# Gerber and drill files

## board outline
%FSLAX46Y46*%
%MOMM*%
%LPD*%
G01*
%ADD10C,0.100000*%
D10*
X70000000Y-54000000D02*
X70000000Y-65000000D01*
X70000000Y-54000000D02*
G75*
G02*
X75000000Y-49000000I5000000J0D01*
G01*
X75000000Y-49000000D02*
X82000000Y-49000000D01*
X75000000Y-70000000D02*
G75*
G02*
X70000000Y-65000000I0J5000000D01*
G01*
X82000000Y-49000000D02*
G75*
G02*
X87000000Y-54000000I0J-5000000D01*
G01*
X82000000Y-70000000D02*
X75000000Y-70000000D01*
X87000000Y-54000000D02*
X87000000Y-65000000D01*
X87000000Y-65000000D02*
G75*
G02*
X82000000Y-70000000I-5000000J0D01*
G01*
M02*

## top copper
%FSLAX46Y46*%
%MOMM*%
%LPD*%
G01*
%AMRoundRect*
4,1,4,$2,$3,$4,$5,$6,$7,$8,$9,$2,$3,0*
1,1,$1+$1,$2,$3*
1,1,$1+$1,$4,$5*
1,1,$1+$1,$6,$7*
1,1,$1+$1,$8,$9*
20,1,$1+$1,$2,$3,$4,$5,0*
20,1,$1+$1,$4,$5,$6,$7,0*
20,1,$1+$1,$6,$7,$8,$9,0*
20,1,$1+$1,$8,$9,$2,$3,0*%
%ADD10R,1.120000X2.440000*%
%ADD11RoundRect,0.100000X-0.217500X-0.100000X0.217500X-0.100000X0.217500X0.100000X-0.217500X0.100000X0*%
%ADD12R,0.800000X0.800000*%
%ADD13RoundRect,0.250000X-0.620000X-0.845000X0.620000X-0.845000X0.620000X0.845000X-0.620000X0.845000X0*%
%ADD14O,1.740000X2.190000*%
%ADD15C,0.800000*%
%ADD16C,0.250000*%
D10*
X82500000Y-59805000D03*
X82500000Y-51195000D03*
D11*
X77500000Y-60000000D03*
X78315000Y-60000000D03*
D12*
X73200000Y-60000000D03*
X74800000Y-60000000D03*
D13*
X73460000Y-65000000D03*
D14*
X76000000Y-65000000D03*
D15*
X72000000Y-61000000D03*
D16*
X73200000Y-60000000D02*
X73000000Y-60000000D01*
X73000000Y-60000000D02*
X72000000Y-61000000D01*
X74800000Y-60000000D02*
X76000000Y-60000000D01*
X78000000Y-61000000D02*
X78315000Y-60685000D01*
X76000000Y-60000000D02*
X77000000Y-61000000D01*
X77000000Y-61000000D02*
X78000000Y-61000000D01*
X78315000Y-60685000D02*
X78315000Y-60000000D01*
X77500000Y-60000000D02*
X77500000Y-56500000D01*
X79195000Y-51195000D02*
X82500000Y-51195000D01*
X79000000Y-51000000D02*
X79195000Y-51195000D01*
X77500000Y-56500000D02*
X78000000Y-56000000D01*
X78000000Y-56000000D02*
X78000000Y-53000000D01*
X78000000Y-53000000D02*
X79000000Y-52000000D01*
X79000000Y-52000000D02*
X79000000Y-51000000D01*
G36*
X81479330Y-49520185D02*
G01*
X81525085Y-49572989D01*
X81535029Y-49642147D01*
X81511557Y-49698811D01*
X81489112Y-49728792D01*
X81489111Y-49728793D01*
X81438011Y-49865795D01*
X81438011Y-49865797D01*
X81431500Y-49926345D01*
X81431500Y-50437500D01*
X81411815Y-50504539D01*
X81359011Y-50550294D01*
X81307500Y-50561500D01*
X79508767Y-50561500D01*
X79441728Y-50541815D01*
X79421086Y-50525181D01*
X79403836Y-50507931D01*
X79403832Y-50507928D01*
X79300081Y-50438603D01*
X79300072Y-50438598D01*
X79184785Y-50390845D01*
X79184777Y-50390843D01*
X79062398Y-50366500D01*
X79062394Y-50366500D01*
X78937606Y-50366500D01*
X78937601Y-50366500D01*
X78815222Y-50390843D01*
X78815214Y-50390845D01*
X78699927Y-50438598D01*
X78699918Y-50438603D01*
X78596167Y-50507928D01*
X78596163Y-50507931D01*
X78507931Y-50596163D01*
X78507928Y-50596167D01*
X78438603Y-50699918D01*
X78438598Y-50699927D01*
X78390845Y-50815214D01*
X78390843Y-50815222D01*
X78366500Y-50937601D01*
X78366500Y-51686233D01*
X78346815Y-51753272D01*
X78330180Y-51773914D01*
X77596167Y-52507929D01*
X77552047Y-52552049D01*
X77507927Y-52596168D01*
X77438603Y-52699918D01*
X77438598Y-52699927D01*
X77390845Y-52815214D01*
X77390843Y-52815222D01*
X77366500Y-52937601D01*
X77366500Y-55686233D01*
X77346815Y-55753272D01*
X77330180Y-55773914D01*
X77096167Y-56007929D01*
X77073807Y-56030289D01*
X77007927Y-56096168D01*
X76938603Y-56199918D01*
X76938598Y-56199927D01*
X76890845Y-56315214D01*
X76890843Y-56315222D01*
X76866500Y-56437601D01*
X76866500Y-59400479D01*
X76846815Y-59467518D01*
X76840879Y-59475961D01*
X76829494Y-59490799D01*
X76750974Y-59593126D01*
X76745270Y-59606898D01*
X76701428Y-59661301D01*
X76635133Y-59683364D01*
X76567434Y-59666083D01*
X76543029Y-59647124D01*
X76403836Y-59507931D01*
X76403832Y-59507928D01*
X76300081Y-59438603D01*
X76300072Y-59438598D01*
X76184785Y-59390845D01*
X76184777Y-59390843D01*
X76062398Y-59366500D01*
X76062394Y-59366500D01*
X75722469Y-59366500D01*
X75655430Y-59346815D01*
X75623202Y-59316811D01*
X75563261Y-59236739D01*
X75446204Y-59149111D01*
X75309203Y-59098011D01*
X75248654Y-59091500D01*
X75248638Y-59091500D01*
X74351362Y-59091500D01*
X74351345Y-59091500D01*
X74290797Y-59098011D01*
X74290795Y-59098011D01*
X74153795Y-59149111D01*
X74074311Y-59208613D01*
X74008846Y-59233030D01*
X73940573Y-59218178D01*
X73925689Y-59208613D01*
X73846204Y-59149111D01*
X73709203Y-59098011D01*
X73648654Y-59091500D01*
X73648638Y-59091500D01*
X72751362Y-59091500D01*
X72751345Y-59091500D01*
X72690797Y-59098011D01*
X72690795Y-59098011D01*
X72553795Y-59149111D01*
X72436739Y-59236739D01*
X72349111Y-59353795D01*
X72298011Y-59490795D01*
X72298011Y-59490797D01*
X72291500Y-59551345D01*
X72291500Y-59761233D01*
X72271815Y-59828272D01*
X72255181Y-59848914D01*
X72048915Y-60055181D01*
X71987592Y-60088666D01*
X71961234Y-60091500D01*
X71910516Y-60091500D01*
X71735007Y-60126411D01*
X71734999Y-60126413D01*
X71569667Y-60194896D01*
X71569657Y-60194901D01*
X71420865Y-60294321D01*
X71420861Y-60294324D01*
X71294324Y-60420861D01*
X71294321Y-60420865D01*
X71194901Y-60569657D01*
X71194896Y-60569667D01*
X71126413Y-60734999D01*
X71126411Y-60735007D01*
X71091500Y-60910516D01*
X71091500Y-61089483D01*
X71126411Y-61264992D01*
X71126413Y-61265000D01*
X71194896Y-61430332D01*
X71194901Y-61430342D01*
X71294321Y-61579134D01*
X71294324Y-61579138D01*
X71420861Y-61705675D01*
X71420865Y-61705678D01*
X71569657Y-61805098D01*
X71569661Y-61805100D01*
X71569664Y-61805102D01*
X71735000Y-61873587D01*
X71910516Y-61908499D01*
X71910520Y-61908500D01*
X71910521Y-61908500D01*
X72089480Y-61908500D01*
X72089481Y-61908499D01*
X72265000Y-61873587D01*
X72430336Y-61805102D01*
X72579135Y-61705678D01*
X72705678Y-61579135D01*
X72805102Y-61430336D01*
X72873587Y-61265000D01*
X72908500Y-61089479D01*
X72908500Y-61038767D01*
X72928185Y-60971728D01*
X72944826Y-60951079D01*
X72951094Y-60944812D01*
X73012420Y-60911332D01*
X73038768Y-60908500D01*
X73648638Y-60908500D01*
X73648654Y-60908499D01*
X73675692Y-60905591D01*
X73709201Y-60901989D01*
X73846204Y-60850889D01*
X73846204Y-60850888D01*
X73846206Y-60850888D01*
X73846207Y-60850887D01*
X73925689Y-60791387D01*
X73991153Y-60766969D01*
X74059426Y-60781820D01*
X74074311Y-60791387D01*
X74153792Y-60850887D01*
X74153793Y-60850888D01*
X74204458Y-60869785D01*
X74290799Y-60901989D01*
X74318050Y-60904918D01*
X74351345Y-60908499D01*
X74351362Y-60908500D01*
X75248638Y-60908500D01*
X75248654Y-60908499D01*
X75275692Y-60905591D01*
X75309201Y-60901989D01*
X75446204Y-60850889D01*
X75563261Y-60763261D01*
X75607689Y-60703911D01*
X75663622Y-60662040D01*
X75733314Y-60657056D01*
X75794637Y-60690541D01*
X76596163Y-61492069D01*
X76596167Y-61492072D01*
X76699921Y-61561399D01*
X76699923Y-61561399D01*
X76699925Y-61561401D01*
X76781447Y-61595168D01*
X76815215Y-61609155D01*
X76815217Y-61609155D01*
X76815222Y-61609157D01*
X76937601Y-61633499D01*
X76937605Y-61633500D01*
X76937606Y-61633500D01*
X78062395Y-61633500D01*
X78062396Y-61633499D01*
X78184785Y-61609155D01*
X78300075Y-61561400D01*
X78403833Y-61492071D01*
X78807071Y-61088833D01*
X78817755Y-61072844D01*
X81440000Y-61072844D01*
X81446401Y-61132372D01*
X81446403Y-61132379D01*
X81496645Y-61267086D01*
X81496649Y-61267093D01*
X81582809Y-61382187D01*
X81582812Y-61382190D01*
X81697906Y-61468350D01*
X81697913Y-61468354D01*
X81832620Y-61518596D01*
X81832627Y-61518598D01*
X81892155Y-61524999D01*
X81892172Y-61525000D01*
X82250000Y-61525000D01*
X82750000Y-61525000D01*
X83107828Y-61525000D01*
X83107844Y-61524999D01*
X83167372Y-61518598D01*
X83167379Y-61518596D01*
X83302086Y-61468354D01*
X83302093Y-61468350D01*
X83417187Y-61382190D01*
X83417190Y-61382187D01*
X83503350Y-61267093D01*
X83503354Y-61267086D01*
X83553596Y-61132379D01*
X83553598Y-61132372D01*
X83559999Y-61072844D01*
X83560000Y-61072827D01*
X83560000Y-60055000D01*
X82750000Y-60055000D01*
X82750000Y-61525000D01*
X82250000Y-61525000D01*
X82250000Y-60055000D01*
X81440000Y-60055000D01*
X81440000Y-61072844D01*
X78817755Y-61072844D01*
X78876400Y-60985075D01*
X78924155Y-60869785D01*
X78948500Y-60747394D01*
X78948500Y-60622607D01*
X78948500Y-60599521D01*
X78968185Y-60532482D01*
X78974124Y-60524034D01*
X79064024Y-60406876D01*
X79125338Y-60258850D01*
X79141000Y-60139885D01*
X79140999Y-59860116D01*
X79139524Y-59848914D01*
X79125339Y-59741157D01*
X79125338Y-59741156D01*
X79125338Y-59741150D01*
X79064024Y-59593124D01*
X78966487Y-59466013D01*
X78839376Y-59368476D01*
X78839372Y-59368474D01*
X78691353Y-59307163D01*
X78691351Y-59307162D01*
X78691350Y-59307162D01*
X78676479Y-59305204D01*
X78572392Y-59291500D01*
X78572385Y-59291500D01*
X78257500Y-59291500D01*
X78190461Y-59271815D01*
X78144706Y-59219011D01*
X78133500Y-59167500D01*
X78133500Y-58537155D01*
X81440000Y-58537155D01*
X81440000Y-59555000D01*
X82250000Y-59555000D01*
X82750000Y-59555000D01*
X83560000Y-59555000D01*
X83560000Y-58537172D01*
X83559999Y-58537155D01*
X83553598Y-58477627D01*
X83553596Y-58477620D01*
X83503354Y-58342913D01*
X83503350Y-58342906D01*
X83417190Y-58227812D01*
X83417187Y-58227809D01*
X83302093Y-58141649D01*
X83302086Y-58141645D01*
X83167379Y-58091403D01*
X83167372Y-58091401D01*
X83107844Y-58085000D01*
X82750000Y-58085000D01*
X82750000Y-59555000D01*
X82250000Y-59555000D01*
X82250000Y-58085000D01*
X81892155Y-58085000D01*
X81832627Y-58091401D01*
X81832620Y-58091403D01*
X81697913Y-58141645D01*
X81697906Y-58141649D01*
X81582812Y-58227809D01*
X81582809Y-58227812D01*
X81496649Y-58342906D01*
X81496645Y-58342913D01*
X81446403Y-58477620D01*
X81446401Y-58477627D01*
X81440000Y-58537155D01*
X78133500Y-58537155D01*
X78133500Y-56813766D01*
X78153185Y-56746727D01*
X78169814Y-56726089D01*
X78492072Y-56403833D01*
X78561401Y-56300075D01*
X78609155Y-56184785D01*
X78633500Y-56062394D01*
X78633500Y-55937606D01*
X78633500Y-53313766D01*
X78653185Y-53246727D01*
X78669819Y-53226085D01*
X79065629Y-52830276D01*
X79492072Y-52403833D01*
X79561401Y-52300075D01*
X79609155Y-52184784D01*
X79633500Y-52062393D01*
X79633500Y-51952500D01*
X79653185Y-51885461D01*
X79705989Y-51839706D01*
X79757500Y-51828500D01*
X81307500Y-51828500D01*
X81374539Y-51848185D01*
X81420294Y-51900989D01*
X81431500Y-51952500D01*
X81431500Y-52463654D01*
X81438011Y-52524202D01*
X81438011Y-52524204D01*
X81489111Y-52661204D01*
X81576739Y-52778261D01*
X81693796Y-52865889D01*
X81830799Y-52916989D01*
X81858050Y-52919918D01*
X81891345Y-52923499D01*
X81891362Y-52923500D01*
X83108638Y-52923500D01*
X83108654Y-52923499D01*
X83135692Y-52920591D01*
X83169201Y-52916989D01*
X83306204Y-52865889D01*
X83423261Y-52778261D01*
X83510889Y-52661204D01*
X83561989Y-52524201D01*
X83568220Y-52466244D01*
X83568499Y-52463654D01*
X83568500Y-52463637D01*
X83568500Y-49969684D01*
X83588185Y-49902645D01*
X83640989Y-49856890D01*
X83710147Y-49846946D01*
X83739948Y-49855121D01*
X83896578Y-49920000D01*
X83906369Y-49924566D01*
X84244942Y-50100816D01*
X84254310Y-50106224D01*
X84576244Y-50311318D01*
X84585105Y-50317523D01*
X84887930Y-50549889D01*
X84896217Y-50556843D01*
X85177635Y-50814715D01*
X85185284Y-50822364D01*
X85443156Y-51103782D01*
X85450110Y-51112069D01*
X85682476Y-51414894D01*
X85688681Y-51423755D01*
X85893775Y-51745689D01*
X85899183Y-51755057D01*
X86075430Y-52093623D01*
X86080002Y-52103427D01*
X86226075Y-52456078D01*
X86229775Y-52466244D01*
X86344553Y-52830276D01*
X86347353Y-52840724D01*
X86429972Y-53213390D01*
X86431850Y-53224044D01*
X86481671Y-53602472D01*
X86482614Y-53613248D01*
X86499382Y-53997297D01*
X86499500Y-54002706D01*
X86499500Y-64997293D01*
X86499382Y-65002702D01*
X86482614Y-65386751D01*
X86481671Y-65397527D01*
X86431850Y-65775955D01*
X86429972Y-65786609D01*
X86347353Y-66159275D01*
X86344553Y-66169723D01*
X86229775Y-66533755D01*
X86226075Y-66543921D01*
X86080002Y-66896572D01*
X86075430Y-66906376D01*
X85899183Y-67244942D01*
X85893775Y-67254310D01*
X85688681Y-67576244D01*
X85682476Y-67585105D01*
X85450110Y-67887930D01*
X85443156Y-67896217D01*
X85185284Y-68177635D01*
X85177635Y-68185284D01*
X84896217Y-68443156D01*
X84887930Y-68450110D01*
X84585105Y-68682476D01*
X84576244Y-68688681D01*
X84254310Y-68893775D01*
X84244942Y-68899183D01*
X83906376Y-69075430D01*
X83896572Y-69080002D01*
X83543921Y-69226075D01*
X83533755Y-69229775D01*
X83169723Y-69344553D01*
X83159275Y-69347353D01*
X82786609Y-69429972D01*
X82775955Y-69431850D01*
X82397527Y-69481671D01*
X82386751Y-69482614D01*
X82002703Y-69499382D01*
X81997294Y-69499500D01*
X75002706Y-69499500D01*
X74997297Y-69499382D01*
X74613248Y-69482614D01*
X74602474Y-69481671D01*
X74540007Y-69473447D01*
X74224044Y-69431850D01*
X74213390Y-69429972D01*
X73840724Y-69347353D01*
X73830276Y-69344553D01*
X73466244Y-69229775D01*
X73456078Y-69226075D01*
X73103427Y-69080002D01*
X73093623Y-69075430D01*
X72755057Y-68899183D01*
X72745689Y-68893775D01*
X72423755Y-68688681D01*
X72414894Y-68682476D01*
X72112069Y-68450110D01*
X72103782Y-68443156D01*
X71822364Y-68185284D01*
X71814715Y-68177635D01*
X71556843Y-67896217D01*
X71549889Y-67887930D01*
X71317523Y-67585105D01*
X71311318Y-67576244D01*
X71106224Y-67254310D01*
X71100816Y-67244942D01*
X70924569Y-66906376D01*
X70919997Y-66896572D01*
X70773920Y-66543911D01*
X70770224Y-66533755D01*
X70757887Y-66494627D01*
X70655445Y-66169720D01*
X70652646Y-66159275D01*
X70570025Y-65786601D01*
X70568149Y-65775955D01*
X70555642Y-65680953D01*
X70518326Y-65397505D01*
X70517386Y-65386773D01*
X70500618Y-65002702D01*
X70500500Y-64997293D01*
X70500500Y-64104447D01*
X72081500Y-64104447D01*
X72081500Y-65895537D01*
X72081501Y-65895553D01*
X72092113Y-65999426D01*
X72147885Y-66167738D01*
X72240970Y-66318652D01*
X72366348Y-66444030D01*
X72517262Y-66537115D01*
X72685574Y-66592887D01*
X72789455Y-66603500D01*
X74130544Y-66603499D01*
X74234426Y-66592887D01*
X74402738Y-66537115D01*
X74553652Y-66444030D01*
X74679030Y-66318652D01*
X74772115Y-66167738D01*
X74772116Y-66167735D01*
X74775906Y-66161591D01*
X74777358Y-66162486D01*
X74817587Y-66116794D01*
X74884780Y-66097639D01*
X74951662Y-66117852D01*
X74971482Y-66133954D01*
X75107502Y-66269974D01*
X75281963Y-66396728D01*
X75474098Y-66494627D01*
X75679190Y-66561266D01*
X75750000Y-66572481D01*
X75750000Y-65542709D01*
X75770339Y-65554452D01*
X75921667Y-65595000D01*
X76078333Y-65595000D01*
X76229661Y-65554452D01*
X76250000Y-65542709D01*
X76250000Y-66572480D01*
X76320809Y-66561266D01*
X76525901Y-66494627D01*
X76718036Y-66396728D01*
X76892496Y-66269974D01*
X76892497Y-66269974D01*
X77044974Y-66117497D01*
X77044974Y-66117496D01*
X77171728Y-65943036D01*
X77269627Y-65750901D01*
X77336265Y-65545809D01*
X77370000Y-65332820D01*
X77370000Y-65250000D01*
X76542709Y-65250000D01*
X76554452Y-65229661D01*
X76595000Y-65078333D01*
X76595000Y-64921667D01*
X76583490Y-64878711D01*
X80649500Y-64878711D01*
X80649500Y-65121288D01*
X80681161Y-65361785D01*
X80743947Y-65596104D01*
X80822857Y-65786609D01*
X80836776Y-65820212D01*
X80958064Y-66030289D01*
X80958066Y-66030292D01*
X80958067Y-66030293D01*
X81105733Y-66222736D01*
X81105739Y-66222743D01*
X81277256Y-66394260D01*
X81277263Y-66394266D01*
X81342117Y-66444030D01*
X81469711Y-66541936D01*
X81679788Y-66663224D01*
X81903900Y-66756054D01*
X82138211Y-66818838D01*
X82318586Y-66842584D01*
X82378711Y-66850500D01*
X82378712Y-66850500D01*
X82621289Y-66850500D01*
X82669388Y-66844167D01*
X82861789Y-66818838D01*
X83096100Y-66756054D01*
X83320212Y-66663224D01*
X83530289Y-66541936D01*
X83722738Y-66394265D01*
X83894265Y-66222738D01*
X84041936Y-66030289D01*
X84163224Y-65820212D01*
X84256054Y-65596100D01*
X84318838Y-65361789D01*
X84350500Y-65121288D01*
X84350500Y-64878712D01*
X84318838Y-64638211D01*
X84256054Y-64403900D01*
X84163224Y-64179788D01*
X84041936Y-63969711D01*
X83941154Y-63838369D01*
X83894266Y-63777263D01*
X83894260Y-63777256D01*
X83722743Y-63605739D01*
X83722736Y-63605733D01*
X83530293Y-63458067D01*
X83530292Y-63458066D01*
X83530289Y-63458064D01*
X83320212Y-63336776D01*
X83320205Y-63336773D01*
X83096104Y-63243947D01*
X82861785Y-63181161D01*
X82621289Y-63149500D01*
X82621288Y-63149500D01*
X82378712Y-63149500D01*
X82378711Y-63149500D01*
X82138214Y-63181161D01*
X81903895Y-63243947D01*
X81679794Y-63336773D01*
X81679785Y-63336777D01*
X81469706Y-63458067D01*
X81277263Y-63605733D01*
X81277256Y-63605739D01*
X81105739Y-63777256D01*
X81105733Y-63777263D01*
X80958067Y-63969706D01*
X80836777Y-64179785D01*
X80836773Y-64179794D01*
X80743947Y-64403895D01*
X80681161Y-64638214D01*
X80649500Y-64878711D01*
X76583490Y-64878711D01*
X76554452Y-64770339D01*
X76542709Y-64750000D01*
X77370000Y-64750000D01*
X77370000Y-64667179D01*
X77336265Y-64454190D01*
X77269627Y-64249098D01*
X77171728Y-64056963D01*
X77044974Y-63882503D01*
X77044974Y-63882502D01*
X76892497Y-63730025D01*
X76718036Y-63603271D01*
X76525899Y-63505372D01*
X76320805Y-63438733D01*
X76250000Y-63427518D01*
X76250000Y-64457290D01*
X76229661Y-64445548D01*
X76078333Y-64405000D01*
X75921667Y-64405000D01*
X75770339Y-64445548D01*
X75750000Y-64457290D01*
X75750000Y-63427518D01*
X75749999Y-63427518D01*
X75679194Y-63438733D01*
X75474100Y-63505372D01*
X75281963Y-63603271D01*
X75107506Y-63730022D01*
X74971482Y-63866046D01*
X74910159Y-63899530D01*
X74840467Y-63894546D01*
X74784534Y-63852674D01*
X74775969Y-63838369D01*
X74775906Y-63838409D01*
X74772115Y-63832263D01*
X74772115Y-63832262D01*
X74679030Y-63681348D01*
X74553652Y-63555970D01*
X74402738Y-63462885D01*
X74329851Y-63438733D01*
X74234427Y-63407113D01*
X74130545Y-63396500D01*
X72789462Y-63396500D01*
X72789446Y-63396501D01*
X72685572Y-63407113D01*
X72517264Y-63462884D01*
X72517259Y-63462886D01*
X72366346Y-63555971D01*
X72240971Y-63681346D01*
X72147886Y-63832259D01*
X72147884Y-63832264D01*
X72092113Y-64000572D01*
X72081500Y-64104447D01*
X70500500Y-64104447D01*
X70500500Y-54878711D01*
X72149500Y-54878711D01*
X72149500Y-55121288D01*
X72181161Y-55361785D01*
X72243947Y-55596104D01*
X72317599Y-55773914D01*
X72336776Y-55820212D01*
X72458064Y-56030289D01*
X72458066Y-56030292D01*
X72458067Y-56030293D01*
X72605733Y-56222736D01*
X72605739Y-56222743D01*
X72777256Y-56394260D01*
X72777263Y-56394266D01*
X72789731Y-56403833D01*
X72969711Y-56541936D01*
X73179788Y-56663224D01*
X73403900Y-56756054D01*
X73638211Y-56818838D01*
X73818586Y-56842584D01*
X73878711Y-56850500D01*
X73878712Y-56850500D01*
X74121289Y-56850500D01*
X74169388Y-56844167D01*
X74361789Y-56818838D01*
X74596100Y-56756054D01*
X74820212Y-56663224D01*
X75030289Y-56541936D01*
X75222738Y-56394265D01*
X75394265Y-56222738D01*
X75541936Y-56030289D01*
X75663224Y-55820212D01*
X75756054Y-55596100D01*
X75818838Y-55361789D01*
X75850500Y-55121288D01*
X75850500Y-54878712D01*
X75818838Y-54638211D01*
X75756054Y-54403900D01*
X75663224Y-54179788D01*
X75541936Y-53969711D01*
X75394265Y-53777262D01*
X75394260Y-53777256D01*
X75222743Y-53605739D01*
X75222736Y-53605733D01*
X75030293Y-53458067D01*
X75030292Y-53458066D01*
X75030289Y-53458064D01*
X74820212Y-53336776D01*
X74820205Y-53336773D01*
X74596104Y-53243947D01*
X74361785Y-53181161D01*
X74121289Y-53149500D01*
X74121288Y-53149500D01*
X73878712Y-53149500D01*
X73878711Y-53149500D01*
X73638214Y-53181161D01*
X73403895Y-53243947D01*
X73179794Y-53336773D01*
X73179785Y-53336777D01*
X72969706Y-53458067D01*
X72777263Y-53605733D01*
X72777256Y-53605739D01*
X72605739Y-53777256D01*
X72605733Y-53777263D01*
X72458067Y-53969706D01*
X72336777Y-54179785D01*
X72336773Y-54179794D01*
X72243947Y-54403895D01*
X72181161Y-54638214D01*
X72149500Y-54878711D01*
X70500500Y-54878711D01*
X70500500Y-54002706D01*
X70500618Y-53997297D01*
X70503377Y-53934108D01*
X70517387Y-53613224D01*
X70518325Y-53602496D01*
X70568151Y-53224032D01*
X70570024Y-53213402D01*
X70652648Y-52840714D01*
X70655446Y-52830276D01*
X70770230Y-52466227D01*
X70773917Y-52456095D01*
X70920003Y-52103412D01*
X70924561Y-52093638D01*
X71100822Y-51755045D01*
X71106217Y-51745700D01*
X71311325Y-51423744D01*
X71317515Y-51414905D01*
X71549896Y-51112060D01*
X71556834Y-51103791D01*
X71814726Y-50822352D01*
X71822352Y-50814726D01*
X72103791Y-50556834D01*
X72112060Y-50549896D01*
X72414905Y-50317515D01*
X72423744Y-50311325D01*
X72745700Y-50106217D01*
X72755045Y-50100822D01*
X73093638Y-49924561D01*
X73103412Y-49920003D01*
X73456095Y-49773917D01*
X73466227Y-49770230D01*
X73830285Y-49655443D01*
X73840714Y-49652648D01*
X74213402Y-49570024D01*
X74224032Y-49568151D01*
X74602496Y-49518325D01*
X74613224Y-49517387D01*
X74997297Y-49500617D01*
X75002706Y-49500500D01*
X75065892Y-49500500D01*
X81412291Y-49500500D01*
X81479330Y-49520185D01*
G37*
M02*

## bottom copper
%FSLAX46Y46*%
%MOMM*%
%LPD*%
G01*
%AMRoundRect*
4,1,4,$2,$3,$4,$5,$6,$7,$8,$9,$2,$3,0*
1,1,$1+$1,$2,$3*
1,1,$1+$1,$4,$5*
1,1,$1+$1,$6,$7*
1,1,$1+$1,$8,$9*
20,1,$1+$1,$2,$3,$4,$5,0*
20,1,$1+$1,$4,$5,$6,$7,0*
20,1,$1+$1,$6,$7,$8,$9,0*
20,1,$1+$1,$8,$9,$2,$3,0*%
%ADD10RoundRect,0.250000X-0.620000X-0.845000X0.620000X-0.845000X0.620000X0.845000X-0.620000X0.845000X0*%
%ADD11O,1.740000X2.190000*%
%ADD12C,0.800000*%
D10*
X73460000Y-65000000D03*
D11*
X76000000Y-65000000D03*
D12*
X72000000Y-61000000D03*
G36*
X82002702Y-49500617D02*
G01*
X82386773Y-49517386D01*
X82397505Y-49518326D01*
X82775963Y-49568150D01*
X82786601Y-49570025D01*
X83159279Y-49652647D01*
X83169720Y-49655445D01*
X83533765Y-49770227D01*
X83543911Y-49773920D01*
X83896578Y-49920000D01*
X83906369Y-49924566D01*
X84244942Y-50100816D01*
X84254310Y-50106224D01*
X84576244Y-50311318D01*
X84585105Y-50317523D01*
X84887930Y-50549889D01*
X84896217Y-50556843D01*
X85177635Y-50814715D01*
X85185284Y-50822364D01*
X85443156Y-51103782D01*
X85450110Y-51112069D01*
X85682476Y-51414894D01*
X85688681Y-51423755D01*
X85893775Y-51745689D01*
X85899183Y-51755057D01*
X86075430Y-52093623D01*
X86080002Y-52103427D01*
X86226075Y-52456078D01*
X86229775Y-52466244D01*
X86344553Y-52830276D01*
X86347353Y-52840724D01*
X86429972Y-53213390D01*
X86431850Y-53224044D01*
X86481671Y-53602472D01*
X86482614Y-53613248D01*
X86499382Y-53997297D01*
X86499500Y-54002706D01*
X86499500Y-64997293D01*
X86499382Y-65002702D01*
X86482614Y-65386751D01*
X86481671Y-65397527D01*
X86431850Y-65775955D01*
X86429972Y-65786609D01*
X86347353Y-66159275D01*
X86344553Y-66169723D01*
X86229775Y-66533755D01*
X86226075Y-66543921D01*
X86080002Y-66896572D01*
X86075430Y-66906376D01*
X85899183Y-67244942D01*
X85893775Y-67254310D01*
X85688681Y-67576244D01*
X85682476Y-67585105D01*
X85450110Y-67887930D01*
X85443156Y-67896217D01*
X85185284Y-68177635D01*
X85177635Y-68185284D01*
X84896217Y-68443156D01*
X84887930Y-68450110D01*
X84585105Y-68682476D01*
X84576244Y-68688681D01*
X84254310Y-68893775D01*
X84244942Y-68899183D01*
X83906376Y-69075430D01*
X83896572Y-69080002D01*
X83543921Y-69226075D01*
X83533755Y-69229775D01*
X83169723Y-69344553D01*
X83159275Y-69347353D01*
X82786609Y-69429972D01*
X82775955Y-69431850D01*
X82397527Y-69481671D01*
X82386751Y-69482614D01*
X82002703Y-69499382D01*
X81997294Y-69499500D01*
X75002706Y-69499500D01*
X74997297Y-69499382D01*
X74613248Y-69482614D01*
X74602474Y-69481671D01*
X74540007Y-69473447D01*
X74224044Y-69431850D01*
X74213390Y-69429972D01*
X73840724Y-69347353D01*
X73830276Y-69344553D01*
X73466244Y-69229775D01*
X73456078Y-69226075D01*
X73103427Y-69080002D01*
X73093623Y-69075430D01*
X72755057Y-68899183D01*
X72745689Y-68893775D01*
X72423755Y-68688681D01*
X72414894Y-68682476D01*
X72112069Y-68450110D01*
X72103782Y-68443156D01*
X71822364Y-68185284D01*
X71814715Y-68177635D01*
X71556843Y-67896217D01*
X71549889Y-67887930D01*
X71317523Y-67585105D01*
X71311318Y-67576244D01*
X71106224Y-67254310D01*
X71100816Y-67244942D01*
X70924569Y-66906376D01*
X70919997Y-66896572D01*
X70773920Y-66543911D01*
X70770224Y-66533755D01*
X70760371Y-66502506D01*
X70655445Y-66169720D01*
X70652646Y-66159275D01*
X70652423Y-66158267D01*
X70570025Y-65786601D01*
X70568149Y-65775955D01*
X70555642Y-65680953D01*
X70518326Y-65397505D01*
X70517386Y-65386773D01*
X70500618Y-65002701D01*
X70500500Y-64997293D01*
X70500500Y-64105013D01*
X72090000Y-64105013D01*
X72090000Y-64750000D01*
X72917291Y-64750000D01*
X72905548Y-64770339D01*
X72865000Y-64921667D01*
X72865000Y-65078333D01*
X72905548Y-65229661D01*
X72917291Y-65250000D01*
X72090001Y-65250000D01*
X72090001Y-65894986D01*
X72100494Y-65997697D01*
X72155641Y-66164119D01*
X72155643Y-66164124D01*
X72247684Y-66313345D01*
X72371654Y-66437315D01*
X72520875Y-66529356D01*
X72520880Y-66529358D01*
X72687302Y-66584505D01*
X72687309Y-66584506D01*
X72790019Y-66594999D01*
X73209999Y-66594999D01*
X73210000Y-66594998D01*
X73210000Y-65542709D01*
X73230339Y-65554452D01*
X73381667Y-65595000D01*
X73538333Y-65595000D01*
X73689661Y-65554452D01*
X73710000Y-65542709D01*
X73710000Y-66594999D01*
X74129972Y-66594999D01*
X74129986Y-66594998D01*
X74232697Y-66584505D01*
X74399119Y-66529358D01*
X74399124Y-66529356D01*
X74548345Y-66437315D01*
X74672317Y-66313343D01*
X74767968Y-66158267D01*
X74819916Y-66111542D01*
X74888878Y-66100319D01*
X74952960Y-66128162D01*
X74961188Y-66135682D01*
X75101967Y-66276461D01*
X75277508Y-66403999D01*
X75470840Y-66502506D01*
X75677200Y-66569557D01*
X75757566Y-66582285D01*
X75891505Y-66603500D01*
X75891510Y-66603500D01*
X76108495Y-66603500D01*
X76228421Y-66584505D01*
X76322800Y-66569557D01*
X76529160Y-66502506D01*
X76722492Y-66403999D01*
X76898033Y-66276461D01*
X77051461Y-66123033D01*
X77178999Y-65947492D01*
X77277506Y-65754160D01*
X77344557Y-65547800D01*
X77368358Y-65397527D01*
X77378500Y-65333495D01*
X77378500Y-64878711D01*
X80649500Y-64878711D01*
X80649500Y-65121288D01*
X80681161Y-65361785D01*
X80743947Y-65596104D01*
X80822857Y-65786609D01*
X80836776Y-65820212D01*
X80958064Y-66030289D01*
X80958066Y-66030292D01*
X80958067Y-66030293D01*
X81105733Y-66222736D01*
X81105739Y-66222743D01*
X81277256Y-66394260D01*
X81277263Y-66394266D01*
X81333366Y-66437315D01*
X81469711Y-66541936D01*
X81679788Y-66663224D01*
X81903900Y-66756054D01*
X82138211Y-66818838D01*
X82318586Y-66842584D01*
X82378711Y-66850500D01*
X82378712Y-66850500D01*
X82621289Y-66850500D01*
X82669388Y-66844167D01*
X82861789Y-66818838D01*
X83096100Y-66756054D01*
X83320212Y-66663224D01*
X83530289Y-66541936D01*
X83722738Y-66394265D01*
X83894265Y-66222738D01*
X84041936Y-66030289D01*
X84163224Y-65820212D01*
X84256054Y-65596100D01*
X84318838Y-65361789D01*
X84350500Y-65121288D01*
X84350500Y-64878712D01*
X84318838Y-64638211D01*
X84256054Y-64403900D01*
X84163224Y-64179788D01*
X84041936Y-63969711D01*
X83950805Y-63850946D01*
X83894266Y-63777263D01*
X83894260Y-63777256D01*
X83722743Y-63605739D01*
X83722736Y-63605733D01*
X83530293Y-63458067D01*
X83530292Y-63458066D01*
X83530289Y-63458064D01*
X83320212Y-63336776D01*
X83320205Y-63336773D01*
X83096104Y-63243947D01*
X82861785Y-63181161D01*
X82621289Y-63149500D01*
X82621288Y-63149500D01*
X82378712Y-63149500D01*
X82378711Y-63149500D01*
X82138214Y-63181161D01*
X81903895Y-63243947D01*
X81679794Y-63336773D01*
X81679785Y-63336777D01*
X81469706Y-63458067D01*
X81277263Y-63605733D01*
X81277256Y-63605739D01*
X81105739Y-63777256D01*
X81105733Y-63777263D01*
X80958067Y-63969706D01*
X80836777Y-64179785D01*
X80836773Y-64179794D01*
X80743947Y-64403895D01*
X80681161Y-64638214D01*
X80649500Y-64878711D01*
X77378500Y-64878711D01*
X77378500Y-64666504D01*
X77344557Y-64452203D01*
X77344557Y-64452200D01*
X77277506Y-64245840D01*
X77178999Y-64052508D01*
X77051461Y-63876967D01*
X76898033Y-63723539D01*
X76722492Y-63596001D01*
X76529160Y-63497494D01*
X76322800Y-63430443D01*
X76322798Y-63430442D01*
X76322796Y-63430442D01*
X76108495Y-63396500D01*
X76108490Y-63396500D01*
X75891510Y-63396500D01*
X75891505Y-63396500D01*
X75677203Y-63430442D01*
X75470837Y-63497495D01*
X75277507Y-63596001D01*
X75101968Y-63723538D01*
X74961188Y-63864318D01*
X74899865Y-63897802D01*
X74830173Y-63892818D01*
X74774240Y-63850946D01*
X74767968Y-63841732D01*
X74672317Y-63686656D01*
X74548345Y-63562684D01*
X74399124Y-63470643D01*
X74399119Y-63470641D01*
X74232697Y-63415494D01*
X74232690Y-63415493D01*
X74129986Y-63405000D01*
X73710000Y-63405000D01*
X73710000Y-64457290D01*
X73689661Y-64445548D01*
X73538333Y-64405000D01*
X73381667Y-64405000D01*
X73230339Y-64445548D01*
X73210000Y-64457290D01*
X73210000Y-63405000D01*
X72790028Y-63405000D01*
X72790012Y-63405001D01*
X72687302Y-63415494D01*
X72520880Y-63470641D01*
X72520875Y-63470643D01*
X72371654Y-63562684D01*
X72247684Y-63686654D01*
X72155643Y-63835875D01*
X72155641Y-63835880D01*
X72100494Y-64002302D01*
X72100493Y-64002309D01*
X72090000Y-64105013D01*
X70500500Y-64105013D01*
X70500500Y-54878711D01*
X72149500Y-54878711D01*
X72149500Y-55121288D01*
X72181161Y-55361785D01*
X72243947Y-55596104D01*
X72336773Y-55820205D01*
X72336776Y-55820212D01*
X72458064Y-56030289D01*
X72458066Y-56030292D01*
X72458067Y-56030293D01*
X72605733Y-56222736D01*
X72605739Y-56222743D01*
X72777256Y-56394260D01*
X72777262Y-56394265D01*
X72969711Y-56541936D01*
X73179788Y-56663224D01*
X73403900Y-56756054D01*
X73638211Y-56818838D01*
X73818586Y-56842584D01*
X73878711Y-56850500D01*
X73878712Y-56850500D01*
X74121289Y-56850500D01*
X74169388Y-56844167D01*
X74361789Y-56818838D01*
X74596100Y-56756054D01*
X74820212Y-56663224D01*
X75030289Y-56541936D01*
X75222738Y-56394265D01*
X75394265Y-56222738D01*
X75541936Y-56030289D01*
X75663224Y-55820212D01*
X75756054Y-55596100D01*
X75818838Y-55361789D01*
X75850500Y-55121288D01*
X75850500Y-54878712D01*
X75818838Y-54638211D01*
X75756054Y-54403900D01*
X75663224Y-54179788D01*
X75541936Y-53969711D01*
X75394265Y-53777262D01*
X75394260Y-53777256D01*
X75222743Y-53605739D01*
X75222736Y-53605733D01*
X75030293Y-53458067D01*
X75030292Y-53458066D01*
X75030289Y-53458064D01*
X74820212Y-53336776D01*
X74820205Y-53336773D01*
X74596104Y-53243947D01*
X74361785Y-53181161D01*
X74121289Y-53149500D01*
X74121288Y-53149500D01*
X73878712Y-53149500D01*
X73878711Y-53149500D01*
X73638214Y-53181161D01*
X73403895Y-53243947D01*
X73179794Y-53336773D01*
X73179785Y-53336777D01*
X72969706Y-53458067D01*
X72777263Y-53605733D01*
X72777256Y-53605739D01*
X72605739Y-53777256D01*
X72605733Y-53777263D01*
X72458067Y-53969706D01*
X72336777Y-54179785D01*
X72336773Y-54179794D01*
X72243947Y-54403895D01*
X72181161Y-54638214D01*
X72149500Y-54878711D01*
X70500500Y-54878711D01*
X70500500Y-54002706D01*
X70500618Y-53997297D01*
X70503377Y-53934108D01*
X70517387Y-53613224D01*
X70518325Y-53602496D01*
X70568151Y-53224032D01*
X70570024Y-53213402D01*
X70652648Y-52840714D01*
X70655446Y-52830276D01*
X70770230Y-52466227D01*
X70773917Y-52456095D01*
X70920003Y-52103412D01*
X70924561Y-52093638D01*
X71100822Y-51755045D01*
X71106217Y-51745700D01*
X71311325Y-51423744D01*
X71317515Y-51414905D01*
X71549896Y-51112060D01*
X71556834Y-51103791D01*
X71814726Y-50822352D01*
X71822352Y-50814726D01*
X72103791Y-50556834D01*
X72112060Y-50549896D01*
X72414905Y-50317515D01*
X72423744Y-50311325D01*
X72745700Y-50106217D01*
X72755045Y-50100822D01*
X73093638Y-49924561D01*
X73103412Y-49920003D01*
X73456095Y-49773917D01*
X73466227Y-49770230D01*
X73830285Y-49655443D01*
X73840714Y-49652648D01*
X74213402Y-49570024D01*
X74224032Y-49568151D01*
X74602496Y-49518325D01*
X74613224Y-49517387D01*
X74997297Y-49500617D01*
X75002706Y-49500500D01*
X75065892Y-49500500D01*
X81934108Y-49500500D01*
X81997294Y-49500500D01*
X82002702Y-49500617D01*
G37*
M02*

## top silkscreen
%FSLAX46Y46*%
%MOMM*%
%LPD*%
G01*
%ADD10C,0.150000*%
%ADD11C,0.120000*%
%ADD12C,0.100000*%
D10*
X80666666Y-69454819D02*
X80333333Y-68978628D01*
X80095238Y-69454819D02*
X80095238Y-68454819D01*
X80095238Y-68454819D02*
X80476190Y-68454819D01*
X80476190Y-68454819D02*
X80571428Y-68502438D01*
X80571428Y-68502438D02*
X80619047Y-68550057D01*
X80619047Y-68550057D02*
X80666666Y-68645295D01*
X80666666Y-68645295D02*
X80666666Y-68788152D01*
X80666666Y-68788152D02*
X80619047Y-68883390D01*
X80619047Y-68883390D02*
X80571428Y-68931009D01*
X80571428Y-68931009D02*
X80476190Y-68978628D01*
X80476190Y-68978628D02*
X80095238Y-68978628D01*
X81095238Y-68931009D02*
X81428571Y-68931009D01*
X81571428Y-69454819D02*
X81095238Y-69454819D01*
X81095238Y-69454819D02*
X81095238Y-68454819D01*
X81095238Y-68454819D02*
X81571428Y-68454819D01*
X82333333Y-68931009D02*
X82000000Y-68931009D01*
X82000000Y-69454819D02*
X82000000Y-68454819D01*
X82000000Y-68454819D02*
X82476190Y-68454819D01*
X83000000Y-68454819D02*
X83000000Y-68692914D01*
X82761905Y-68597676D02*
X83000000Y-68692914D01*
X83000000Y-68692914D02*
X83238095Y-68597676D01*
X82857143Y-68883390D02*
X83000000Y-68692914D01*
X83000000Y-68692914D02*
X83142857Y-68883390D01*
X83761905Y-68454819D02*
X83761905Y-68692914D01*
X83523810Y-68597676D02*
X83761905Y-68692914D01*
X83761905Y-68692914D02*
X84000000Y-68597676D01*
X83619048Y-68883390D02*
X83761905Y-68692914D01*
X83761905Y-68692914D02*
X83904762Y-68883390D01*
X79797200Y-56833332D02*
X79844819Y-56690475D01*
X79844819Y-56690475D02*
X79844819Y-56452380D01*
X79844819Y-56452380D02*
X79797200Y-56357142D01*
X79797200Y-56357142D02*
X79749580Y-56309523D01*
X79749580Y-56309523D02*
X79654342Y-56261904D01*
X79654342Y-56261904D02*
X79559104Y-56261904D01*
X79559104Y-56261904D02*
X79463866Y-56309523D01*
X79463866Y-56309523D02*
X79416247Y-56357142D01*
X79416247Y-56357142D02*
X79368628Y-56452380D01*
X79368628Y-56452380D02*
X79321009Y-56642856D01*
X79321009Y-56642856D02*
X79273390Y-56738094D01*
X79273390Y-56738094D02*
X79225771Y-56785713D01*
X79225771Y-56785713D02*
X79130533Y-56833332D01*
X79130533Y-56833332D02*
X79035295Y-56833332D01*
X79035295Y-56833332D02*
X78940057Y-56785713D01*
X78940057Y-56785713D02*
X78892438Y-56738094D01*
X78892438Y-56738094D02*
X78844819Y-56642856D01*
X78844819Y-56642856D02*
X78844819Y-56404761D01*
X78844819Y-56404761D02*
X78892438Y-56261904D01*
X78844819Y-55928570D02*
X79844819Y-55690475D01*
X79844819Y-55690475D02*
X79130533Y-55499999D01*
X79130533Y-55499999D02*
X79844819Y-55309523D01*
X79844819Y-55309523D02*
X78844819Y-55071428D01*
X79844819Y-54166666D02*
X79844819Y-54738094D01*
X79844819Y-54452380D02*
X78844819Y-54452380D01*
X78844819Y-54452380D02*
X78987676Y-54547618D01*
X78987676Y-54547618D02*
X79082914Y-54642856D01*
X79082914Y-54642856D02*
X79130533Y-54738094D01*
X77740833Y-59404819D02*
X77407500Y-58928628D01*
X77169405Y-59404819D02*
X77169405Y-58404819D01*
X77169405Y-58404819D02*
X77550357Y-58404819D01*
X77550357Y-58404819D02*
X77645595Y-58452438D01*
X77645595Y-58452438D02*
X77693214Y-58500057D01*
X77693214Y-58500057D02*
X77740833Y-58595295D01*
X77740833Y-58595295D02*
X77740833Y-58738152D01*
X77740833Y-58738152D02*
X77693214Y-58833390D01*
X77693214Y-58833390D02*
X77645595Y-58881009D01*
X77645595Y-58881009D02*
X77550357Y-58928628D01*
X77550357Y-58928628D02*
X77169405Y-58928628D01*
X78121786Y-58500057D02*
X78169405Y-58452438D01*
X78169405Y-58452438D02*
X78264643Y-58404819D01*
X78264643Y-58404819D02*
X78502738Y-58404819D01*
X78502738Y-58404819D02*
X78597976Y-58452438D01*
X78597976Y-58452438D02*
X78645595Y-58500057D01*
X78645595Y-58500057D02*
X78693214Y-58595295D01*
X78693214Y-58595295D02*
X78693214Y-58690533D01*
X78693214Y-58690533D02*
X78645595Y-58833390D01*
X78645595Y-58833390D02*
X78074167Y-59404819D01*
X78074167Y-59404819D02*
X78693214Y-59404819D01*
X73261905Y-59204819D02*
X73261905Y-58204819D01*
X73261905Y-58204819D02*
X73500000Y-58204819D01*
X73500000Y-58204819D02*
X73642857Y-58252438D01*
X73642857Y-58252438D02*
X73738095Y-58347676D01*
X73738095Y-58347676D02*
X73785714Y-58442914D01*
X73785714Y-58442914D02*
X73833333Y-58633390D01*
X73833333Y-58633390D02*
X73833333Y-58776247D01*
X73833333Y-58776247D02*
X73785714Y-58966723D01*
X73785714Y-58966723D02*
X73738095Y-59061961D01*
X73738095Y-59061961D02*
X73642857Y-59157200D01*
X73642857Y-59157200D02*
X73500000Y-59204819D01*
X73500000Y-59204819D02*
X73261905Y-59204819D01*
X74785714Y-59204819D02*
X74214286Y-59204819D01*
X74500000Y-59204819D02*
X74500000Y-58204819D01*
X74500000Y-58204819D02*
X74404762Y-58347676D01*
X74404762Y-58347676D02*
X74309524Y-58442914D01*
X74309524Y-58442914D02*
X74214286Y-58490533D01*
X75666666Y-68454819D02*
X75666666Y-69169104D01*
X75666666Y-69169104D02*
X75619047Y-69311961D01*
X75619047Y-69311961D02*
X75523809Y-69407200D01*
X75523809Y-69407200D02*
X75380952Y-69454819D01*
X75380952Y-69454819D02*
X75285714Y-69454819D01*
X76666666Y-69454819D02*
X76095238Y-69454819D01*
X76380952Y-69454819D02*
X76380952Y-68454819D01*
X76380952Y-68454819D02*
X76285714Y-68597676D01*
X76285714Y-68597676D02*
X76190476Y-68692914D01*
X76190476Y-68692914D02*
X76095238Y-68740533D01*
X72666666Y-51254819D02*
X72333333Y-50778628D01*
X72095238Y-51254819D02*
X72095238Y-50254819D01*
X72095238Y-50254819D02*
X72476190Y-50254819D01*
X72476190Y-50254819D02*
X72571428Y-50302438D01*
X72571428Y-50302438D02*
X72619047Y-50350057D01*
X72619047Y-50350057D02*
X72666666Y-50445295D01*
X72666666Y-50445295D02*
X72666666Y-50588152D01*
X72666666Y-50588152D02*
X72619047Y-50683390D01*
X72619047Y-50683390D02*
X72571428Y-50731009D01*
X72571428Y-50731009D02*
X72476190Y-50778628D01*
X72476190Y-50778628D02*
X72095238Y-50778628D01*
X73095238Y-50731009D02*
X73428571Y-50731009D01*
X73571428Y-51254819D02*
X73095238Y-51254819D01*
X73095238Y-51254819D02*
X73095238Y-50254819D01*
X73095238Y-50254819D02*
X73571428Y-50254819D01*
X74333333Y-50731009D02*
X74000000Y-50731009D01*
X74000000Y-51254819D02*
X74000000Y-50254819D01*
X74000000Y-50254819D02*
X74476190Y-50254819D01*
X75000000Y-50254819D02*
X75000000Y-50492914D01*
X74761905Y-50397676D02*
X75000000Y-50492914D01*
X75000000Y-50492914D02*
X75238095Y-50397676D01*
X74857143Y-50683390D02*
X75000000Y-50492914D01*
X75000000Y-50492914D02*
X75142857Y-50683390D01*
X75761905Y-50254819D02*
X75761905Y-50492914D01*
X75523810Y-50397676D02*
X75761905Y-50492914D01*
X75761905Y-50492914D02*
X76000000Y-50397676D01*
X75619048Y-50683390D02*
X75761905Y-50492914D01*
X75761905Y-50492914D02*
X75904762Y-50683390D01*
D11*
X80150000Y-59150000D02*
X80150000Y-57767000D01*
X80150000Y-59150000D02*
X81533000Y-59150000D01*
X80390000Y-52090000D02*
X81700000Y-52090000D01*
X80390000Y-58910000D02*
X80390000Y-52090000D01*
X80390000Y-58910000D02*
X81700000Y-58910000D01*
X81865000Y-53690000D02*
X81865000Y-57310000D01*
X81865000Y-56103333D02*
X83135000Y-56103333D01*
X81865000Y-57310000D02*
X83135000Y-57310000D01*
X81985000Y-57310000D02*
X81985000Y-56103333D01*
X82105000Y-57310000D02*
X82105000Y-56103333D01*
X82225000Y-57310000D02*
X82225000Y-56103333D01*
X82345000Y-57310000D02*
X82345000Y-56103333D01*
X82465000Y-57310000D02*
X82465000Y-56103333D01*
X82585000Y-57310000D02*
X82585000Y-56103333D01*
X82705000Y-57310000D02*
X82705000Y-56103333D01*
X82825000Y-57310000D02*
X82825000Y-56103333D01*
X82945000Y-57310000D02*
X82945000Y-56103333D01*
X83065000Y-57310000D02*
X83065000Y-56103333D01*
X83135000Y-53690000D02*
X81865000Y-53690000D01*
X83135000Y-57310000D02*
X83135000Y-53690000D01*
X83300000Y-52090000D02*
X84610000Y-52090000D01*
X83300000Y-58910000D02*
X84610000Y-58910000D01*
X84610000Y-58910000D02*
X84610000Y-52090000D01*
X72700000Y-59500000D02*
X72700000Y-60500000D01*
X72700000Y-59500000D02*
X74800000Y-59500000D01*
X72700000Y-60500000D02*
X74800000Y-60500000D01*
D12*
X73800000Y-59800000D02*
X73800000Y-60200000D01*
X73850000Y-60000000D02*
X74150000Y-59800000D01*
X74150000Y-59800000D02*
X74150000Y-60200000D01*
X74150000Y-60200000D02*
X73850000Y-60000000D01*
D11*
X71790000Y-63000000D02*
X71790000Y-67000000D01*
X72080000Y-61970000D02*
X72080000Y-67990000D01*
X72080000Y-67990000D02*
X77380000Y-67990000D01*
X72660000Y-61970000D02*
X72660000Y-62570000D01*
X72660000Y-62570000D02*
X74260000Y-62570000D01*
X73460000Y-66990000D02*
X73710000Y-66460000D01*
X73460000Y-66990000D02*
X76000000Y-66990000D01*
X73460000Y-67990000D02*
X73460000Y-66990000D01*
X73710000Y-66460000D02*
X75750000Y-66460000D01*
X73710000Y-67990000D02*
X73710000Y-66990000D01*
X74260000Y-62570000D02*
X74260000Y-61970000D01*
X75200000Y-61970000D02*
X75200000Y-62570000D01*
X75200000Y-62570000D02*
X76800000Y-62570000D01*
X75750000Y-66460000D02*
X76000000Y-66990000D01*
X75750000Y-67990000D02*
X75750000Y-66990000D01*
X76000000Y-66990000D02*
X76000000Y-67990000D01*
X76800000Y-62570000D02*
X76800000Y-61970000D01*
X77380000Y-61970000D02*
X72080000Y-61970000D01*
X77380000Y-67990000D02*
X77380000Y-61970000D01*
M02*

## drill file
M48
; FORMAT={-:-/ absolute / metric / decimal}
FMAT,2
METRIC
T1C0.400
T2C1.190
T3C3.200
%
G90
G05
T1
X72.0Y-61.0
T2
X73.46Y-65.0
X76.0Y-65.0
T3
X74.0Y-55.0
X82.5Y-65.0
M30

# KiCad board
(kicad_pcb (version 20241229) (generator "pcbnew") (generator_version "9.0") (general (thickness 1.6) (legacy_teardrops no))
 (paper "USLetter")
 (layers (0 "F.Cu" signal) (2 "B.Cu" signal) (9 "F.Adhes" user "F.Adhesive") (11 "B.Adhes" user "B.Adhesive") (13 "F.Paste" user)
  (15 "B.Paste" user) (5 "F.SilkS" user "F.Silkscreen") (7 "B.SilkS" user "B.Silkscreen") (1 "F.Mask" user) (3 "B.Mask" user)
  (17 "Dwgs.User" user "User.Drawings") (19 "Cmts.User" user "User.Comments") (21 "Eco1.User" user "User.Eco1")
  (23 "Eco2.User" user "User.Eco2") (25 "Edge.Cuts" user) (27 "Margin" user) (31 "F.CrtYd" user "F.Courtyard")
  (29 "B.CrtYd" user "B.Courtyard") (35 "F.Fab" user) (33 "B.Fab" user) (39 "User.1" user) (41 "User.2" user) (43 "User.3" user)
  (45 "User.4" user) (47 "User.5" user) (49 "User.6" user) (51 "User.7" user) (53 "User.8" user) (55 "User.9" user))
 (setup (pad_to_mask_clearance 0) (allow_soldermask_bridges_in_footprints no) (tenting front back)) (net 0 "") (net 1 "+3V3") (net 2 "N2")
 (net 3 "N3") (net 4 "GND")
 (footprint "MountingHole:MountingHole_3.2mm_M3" (layer "F.Cu") (at 82.5 65)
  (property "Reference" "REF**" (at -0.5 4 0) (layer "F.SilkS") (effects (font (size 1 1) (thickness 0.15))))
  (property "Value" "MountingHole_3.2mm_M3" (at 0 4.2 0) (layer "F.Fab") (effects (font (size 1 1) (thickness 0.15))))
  (pad "" np_thru_hole circle (at 0 0) (size 3.2 3.2) (drill 3.2) (layers "*.Cu" "*.Mask")))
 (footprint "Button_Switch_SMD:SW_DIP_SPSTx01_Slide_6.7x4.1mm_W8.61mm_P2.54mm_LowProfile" (layer "F.Cu") (at 82.5 55.5 90)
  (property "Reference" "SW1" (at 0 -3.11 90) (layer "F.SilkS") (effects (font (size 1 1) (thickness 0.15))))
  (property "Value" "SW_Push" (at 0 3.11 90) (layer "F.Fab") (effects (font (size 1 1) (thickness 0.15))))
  (fp_line (start -3.65 -2.35) (end -2.267 -2.35) (stroke (width 0.12) (type solid)) (layer "F.SilkS"))
  (fp_line (start -3.65 -2.35) (end -3.65 -0.967) (stroke (width 0.12) (type solid)) (layer "F.SilkS"))
  (fp_line (start 3.41 -2.11) (end 3.41 -0.8) (stroke (width 0.12) (type solid)) (layer "F.SilkS"))
  (fp_line (start -3.41 -2.11) (end 3.41 -2.11) (stroke (width 0.12) (type solid)) (layer "F.SilkS"))
  (fp_line (start -3.41 -2.11) (end -3.41 -0.8) (stroke (width 0.12) (type solid)) (layer "F.SilkS"))
  (fp_line (start 1.81 -0.635) (end -1.81 -0.635) (stroke (width 0.12) (type solid)) (layer "F.SilkS"))
  (fp_line (start -0.603333 -0.635) (end -0.603333 0.635) (stroke (width 0.12) (type solid)) (layer "F.SilkS"))
  (fp_line (start -1.81 -0.635) (end -1.81 0.635) (stroke (width 0.12) (type solid)) (layer "F.SilkS"))
  (fp_line (start -1.81 -0.515) (end -0.603333 -0.515) (stroke (width 0.12) (type solid)) (layer "F.SilkS"))
  (fp_line (start -1.81 -0.395) (end -0.603333 -0.395) (stroke (width 0.12) (type solid)) (layer "F.SilkS"))
  (fp_line (start -1.81 -0.275) (end -0.603333 -0.275) (stroke (width 0.12) (type solid)) (layer "F.SilkS"))
  (fp_line (start -1.81 -0.155) (end -0.603333 -0.155) (stroke (width 0.12) (type solid)) (layer "F.SilkS"))
  (fp_line (start -1.81 -0.035) (end -0.603333 -0.035) (stroke (width 0.12) (type solid)) (layer "F.SilkS"))
  (fp_line (start -1.81 0.085) (end -0.603333 0.085) (stroke (width 0.12) (type solid)) (layer "F.SilkS"))
  (fp_line (start -1.81 0.205) (end -0.603333 0.205) (stroke (width 0.12) (type solid)) (layer "F.SilkS"))
  (fp_line (start -1.81 0.325) (end -0.603333 0.325) (stroke (width 0.12) (type solid)) (layer "F.SilkS"))
  (fp_line (start -1.81 0.445) (end -0.603333 0.445) (stroke (width 0.12) (type solid)) (layer "F.SilkS"))
  (fp_line (start -1.81 0.565) (end -0.603333 0.565) (stroke (width 0.12) (type solid)) (layer "F.SilkS"))
  (fp_line (start 1.81 0.635) (end 1.81 -0.635) (stroke (width 0.12) (type solid)) (layer "F.SilkS"))
  (fp_line (start -1.81 0.635) (end 1.81 0.635) (stroke (width 0.12) (type solid)) (layer "F.SilkS"))
  (fp_line (start 3.41 0.8) (end 3.41 2.11) (stroke (width 0.12) (type solid)) (layer "F.SilkS"))
  (fp_line (start -3.41 0.8) (end -3.41 2.11) (stroke (width 0.12) (type solid)) (layer "F.SilkS"))
  (fp_line (start -3.41 2.11) (end 3.41 2.11) (stroke (width 0.12) (type solid)) (layer "F.SilkS"))
  (pad "1" smd rect (at -4.305 0 90) (size 2.44 1.12) (layers "F.Cu" "F.Mask" "F.Paste") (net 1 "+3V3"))
  (pad "2" smd rect (at 4.305 0 90) (size 2.44 1.12) (layers "F.Cu" "F.Mask" "F.Paste") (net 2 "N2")))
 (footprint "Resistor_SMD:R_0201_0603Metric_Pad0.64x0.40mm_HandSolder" (layer "F.Cu") (at 77.9075 60)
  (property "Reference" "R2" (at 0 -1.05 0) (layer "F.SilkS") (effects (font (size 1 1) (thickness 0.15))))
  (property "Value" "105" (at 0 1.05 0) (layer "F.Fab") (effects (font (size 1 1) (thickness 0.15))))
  (pad "" smd roundrect (at -0.4325 0) (size 0.458 0.36) (layers "F.Paste") (roundrect_rratio 0.25))
  (pad "" smd roundrect (at 0.4325 0) (size 0.458 0.36) (layers "F.Paste") (roundrect_rratio 0.25))
  (pad "1" smd roundrect (at -0.4075 0) (size 0.635 0.4) (layers "F.Cu" "F.Mask") (roundrect_rratio 0.25) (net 2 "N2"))
  (pad "2" smd roundrect (at 0.4075 0) (size 0.635 0.4) (layers "F.Cu" "F.Mask") (roundrect_rratio 0.25) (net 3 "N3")))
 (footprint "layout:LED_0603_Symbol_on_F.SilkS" (layer "F.Cu") (at 74 60)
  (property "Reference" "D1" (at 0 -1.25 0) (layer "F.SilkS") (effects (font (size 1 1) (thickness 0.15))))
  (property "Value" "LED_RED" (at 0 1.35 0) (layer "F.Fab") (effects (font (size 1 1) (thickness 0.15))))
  (fp_line (start -1.3 -0.5) (end -1.3 0.5) (stroke (width 0.12) (type solid)) (layer "F.SilkS"))
  (fp_line (start -1.3 -0.5) (end 0.8 -0.5) (stroke (width 0.12) (type solid)) (layer "F.SilkS"))
  (fp_line (start -1.3 0.5) (end 0.8 0.5) (stroke (width 0.12) (type solid)) (layer "F.SilkS"))
  (fp_line (start -0.2 -0.2) (end -0.2 0.2) (stroke (width 0.1) (type solid)) (layer "F.SilkS"))
  (fp_line (start -0.15 0) (end 0.15 -0.2) (stroke (width 0.1) (type solid)) (layer "F.SilkS"))
  (fp_line (start 0.15 -0.2) (end 0.15 0.2) (stroke (width 0.1) (type solid)) (layer "F.SilkS"))
  (fp_line (start 0.15 0.2) (end -0.15 0) (stroke (width 0.1) (type solid)) (layer "F.SilkS"))
  (pad "1" smd rect (at -0.8 0 180) (size 0.8 0.8) (layers "F.Cu" "F.Mask" "F.Paste") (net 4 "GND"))
  (pad "2" smd rect (at 0.8 0 180) (size 0.8 0.8) (layers "F.Cu" "F.Mask" "F.Paste") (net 3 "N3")))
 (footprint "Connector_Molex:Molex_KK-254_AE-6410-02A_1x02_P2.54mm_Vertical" (layer "F.Cu") (at 73.46 65)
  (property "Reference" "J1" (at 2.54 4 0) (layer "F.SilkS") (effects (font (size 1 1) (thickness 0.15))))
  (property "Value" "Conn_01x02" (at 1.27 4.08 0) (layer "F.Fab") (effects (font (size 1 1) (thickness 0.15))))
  (fp_line (start -1.67 -2) (end -1.67 2) (stroke (width 0.12) (type solid)) (layer "F.SilkS"))
  (fp_line (start -1.38 -3.03) (end -1.38 2.99) (stroke (width 0.12) (type solid)) (layer "F.SilkS"))
  (fp_line (start -1.38 2.99) (end 3.92 2.99) (stroke (width 0.12) (type solid)) (layer "F.SilkS"))
  (fp_line (start -0.8 -3.03) (end -0.8 -2.43) (stroke (width 0.12) (type solid)) (layer "F.SilkS"))
  (fp_line (start -0.8 -2.43) (end 0.8 -2.43) (stroke (width 0.12) (type solid)) (layer "F.SilkS"))
  (fp_line (start 0 1.99) (end 0.25 1.46) (stroke (width 0.12) (type solid)) (layer "F.SilkS"))
  (fp_line (start 0 1.99) (end 2.54 1.99) (stroke (width 0.12) (type solid)) (layer "F.SilkS"))
  (fp_line (start 0 2.99) (end 0 1.99) (stroke (width 0.12) (type solid)) (layer "F.SilkS"))
  (fp_line (start 0.25 1.46) (end 2.29 1.46) (stroke (width 0.12) (type solid)) (layer "F.SilkS"))
  (fp_line (start 0.25 2.99) (end 0.25 1.99) (stroke (width 0.12) (type solid)) (layer "F.SilkS"))
  (fp_line (start 0.8 -2.43) (end 0.8 -3.03) (stroke (width 0.12) (type solid)) (layer "F.SilkS"))
  (fp_line (start 1.74 -3.03) (end 1.74 -2.43) (stroke (width 0.12) (type solid)) (layer "F.SilkS"))
  (fp_line (start 1.74 -2.43) (end 3.34 -2.43) (stroke (width 0.12) (type solid)) (layer "F.SilkS"))
  (fp_line (start 2.29 1.46) (end 2.54 1.99) (stroke (width 0.12) (type solid)) (layer "F.SilkS"))
  (fp_line (start 2.29 2.99) (end 2.29 1.99) (stroke (width 0.12) (type solid)) (layer "F.SilkS"))
  (fp_line (start 2.54 1.99) (end 2.54 2.99) (stroke (width 0.12) (type solid)) (layer "F.SilkS"))
  (fp_line (start 3.34 -2.43) (end 3.34 -3.03) (stroke (width 0.12) (type solid)) (layer "F.SilkS"))
  (fp_line (start 3.92 -3.03) (end -1.38 -3.03) (stroke (width 0.12) (type solid)) (layer "F.SilkS"))
  (fp_line (start 3.92 2.99) (end 3.92 -3.03) (stroke (width 0.12) (type solid)) (layer "F.SilkS"))
  (pad "1" thru_hole roundrect (at 0 0) (size 1.74 2.19) (drill 1.19) (layers "*.Cu" "*.Mask") (remove_unused_layers no)
   (roundrect_rratio 0.143678) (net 4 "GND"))
  (pad "2" thru_hole oval (at 2.54 0) (size 1.74 2.19) (drill 1.19) (layers "*.Cu" "*.Mask") (remove_unused_layers no) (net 1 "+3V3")))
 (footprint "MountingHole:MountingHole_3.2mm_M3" (layer "F.Cu") (at 74 55)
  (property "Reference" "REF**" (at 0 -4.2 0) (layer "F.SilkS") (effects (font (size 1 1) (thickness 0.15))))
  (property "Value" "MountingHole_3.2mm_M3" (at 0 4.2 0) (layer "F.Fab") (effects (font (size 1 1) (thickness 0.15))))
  (pad "" np_thru_hole circle (at 0 0) (size 3.2 3.2) (drill 3.2) (layers "*.Cu" "*.Mask")))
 (gr_line (start 70 54) (end 70 65) (stroke (width 0.1) (type default)) (layer "Edge.Cuts"))
 (gr_arc (start 70 54) (mid 71.464466 50.464466) (end 75 49) (stroke (width 0.1) (type default)) (layer "Edge.Cuts"))
 (gr_line (start 75 49) (end 82 49) (stroke (width 0.1) (type default)) (layer "Edge.Cuts"))
 (gr_arc (start 75 70) (mid 71.464466 68.535534) (end 70 65) (stroke (width 0.1) (type default)) (layer "Edge.Cuts"))
 (gr_arc (start 82 49) (mid 85.535534 50.464466) (end 87 54) (stroke (width 0.1) (type default)) (layer "Edge.Cuts"))
 (gr_line (start 82 70) (end 75 70) (stroke (width 0.1) (type default)) (layer "Edge.Cuts"))
 (gr_line (start 87 54) (end 87 65) (stroke (width 0.1) (type default)) (layer "Edge.Cuts"))
 (gr_arc (start 87 65) (mid 85.535534 68.535534) (end 82 70) (stroke (width 0.1) (type default)) (layer "Edge.Cuts"))
 (segment (start 73.2 60) (end 73 60) (width 0.25) (layer "F.Cu") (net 4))
 (segment (start 73 60) (end 72 61) (width 0.25) (layer "F.Cu") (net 4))
 (via (at 72 61) (size 0.8) (drill 0.4) (layers "F.Cu" "B.Cu") (free yes) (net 4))
 (segment (start 74.8 60) (end 76 60) (width 0.25) (layer "F.Cu") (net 3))
 (segment (start 78 61) (end 78.315 60.685) (width 0.25) (layer "F.Cu") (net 3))
 (segment (start 76 60) (end 77 61) (width 0.25) (layer "F.Cu") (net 3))
 (segment (start 77 61) (end 78 61) (width 0.25) (layer "F.Cu") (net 3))
 (segment (start 78.315 60.685) (end 78.315 60) (width 0.25) (layer "F.Cu") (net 3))
 (segment (start 77.5 60) (end 77.5 56.5) (width 0.25) (layer "F.Cu") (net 2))
 (segment (start 79.195 51.195) (end 82.5 51.195) (width 0.25) (layer "F.Cu") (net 2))
 (segment (start 79 51) (end 79.195 51.195) (width 0.25) (layer "F.Cu") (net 2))
 (segment (start 77.5 56.5) (end 78 56) (width 0.25) (layer "F.Cu") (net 2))
 (segment (start 78 56) (end 78 53) (width 0.25) (layer "F.Cu") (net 2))
 (segment (start 78 53) (end 79 52) (width 0.25) (layer "F.Cu") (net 2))
 (segment (start 79 52) (end 79 51) (width 0.25) (layer "F.Cu") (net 2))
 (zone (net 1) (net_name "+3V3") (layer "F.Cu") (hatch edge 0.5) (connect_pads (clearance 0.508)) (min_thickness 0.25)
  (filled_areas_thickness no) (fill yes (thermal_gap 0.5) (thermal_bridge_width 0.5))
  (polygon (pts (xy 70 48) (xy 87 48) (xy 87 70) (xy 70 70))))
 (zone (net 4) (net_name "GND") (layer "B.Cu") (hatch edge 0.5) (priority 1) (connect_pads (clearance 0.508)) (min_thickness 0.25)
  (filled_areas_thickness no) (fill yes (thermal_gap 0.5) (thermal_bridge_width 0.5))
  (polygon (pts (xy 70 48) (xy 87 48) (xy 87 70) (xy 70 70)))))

